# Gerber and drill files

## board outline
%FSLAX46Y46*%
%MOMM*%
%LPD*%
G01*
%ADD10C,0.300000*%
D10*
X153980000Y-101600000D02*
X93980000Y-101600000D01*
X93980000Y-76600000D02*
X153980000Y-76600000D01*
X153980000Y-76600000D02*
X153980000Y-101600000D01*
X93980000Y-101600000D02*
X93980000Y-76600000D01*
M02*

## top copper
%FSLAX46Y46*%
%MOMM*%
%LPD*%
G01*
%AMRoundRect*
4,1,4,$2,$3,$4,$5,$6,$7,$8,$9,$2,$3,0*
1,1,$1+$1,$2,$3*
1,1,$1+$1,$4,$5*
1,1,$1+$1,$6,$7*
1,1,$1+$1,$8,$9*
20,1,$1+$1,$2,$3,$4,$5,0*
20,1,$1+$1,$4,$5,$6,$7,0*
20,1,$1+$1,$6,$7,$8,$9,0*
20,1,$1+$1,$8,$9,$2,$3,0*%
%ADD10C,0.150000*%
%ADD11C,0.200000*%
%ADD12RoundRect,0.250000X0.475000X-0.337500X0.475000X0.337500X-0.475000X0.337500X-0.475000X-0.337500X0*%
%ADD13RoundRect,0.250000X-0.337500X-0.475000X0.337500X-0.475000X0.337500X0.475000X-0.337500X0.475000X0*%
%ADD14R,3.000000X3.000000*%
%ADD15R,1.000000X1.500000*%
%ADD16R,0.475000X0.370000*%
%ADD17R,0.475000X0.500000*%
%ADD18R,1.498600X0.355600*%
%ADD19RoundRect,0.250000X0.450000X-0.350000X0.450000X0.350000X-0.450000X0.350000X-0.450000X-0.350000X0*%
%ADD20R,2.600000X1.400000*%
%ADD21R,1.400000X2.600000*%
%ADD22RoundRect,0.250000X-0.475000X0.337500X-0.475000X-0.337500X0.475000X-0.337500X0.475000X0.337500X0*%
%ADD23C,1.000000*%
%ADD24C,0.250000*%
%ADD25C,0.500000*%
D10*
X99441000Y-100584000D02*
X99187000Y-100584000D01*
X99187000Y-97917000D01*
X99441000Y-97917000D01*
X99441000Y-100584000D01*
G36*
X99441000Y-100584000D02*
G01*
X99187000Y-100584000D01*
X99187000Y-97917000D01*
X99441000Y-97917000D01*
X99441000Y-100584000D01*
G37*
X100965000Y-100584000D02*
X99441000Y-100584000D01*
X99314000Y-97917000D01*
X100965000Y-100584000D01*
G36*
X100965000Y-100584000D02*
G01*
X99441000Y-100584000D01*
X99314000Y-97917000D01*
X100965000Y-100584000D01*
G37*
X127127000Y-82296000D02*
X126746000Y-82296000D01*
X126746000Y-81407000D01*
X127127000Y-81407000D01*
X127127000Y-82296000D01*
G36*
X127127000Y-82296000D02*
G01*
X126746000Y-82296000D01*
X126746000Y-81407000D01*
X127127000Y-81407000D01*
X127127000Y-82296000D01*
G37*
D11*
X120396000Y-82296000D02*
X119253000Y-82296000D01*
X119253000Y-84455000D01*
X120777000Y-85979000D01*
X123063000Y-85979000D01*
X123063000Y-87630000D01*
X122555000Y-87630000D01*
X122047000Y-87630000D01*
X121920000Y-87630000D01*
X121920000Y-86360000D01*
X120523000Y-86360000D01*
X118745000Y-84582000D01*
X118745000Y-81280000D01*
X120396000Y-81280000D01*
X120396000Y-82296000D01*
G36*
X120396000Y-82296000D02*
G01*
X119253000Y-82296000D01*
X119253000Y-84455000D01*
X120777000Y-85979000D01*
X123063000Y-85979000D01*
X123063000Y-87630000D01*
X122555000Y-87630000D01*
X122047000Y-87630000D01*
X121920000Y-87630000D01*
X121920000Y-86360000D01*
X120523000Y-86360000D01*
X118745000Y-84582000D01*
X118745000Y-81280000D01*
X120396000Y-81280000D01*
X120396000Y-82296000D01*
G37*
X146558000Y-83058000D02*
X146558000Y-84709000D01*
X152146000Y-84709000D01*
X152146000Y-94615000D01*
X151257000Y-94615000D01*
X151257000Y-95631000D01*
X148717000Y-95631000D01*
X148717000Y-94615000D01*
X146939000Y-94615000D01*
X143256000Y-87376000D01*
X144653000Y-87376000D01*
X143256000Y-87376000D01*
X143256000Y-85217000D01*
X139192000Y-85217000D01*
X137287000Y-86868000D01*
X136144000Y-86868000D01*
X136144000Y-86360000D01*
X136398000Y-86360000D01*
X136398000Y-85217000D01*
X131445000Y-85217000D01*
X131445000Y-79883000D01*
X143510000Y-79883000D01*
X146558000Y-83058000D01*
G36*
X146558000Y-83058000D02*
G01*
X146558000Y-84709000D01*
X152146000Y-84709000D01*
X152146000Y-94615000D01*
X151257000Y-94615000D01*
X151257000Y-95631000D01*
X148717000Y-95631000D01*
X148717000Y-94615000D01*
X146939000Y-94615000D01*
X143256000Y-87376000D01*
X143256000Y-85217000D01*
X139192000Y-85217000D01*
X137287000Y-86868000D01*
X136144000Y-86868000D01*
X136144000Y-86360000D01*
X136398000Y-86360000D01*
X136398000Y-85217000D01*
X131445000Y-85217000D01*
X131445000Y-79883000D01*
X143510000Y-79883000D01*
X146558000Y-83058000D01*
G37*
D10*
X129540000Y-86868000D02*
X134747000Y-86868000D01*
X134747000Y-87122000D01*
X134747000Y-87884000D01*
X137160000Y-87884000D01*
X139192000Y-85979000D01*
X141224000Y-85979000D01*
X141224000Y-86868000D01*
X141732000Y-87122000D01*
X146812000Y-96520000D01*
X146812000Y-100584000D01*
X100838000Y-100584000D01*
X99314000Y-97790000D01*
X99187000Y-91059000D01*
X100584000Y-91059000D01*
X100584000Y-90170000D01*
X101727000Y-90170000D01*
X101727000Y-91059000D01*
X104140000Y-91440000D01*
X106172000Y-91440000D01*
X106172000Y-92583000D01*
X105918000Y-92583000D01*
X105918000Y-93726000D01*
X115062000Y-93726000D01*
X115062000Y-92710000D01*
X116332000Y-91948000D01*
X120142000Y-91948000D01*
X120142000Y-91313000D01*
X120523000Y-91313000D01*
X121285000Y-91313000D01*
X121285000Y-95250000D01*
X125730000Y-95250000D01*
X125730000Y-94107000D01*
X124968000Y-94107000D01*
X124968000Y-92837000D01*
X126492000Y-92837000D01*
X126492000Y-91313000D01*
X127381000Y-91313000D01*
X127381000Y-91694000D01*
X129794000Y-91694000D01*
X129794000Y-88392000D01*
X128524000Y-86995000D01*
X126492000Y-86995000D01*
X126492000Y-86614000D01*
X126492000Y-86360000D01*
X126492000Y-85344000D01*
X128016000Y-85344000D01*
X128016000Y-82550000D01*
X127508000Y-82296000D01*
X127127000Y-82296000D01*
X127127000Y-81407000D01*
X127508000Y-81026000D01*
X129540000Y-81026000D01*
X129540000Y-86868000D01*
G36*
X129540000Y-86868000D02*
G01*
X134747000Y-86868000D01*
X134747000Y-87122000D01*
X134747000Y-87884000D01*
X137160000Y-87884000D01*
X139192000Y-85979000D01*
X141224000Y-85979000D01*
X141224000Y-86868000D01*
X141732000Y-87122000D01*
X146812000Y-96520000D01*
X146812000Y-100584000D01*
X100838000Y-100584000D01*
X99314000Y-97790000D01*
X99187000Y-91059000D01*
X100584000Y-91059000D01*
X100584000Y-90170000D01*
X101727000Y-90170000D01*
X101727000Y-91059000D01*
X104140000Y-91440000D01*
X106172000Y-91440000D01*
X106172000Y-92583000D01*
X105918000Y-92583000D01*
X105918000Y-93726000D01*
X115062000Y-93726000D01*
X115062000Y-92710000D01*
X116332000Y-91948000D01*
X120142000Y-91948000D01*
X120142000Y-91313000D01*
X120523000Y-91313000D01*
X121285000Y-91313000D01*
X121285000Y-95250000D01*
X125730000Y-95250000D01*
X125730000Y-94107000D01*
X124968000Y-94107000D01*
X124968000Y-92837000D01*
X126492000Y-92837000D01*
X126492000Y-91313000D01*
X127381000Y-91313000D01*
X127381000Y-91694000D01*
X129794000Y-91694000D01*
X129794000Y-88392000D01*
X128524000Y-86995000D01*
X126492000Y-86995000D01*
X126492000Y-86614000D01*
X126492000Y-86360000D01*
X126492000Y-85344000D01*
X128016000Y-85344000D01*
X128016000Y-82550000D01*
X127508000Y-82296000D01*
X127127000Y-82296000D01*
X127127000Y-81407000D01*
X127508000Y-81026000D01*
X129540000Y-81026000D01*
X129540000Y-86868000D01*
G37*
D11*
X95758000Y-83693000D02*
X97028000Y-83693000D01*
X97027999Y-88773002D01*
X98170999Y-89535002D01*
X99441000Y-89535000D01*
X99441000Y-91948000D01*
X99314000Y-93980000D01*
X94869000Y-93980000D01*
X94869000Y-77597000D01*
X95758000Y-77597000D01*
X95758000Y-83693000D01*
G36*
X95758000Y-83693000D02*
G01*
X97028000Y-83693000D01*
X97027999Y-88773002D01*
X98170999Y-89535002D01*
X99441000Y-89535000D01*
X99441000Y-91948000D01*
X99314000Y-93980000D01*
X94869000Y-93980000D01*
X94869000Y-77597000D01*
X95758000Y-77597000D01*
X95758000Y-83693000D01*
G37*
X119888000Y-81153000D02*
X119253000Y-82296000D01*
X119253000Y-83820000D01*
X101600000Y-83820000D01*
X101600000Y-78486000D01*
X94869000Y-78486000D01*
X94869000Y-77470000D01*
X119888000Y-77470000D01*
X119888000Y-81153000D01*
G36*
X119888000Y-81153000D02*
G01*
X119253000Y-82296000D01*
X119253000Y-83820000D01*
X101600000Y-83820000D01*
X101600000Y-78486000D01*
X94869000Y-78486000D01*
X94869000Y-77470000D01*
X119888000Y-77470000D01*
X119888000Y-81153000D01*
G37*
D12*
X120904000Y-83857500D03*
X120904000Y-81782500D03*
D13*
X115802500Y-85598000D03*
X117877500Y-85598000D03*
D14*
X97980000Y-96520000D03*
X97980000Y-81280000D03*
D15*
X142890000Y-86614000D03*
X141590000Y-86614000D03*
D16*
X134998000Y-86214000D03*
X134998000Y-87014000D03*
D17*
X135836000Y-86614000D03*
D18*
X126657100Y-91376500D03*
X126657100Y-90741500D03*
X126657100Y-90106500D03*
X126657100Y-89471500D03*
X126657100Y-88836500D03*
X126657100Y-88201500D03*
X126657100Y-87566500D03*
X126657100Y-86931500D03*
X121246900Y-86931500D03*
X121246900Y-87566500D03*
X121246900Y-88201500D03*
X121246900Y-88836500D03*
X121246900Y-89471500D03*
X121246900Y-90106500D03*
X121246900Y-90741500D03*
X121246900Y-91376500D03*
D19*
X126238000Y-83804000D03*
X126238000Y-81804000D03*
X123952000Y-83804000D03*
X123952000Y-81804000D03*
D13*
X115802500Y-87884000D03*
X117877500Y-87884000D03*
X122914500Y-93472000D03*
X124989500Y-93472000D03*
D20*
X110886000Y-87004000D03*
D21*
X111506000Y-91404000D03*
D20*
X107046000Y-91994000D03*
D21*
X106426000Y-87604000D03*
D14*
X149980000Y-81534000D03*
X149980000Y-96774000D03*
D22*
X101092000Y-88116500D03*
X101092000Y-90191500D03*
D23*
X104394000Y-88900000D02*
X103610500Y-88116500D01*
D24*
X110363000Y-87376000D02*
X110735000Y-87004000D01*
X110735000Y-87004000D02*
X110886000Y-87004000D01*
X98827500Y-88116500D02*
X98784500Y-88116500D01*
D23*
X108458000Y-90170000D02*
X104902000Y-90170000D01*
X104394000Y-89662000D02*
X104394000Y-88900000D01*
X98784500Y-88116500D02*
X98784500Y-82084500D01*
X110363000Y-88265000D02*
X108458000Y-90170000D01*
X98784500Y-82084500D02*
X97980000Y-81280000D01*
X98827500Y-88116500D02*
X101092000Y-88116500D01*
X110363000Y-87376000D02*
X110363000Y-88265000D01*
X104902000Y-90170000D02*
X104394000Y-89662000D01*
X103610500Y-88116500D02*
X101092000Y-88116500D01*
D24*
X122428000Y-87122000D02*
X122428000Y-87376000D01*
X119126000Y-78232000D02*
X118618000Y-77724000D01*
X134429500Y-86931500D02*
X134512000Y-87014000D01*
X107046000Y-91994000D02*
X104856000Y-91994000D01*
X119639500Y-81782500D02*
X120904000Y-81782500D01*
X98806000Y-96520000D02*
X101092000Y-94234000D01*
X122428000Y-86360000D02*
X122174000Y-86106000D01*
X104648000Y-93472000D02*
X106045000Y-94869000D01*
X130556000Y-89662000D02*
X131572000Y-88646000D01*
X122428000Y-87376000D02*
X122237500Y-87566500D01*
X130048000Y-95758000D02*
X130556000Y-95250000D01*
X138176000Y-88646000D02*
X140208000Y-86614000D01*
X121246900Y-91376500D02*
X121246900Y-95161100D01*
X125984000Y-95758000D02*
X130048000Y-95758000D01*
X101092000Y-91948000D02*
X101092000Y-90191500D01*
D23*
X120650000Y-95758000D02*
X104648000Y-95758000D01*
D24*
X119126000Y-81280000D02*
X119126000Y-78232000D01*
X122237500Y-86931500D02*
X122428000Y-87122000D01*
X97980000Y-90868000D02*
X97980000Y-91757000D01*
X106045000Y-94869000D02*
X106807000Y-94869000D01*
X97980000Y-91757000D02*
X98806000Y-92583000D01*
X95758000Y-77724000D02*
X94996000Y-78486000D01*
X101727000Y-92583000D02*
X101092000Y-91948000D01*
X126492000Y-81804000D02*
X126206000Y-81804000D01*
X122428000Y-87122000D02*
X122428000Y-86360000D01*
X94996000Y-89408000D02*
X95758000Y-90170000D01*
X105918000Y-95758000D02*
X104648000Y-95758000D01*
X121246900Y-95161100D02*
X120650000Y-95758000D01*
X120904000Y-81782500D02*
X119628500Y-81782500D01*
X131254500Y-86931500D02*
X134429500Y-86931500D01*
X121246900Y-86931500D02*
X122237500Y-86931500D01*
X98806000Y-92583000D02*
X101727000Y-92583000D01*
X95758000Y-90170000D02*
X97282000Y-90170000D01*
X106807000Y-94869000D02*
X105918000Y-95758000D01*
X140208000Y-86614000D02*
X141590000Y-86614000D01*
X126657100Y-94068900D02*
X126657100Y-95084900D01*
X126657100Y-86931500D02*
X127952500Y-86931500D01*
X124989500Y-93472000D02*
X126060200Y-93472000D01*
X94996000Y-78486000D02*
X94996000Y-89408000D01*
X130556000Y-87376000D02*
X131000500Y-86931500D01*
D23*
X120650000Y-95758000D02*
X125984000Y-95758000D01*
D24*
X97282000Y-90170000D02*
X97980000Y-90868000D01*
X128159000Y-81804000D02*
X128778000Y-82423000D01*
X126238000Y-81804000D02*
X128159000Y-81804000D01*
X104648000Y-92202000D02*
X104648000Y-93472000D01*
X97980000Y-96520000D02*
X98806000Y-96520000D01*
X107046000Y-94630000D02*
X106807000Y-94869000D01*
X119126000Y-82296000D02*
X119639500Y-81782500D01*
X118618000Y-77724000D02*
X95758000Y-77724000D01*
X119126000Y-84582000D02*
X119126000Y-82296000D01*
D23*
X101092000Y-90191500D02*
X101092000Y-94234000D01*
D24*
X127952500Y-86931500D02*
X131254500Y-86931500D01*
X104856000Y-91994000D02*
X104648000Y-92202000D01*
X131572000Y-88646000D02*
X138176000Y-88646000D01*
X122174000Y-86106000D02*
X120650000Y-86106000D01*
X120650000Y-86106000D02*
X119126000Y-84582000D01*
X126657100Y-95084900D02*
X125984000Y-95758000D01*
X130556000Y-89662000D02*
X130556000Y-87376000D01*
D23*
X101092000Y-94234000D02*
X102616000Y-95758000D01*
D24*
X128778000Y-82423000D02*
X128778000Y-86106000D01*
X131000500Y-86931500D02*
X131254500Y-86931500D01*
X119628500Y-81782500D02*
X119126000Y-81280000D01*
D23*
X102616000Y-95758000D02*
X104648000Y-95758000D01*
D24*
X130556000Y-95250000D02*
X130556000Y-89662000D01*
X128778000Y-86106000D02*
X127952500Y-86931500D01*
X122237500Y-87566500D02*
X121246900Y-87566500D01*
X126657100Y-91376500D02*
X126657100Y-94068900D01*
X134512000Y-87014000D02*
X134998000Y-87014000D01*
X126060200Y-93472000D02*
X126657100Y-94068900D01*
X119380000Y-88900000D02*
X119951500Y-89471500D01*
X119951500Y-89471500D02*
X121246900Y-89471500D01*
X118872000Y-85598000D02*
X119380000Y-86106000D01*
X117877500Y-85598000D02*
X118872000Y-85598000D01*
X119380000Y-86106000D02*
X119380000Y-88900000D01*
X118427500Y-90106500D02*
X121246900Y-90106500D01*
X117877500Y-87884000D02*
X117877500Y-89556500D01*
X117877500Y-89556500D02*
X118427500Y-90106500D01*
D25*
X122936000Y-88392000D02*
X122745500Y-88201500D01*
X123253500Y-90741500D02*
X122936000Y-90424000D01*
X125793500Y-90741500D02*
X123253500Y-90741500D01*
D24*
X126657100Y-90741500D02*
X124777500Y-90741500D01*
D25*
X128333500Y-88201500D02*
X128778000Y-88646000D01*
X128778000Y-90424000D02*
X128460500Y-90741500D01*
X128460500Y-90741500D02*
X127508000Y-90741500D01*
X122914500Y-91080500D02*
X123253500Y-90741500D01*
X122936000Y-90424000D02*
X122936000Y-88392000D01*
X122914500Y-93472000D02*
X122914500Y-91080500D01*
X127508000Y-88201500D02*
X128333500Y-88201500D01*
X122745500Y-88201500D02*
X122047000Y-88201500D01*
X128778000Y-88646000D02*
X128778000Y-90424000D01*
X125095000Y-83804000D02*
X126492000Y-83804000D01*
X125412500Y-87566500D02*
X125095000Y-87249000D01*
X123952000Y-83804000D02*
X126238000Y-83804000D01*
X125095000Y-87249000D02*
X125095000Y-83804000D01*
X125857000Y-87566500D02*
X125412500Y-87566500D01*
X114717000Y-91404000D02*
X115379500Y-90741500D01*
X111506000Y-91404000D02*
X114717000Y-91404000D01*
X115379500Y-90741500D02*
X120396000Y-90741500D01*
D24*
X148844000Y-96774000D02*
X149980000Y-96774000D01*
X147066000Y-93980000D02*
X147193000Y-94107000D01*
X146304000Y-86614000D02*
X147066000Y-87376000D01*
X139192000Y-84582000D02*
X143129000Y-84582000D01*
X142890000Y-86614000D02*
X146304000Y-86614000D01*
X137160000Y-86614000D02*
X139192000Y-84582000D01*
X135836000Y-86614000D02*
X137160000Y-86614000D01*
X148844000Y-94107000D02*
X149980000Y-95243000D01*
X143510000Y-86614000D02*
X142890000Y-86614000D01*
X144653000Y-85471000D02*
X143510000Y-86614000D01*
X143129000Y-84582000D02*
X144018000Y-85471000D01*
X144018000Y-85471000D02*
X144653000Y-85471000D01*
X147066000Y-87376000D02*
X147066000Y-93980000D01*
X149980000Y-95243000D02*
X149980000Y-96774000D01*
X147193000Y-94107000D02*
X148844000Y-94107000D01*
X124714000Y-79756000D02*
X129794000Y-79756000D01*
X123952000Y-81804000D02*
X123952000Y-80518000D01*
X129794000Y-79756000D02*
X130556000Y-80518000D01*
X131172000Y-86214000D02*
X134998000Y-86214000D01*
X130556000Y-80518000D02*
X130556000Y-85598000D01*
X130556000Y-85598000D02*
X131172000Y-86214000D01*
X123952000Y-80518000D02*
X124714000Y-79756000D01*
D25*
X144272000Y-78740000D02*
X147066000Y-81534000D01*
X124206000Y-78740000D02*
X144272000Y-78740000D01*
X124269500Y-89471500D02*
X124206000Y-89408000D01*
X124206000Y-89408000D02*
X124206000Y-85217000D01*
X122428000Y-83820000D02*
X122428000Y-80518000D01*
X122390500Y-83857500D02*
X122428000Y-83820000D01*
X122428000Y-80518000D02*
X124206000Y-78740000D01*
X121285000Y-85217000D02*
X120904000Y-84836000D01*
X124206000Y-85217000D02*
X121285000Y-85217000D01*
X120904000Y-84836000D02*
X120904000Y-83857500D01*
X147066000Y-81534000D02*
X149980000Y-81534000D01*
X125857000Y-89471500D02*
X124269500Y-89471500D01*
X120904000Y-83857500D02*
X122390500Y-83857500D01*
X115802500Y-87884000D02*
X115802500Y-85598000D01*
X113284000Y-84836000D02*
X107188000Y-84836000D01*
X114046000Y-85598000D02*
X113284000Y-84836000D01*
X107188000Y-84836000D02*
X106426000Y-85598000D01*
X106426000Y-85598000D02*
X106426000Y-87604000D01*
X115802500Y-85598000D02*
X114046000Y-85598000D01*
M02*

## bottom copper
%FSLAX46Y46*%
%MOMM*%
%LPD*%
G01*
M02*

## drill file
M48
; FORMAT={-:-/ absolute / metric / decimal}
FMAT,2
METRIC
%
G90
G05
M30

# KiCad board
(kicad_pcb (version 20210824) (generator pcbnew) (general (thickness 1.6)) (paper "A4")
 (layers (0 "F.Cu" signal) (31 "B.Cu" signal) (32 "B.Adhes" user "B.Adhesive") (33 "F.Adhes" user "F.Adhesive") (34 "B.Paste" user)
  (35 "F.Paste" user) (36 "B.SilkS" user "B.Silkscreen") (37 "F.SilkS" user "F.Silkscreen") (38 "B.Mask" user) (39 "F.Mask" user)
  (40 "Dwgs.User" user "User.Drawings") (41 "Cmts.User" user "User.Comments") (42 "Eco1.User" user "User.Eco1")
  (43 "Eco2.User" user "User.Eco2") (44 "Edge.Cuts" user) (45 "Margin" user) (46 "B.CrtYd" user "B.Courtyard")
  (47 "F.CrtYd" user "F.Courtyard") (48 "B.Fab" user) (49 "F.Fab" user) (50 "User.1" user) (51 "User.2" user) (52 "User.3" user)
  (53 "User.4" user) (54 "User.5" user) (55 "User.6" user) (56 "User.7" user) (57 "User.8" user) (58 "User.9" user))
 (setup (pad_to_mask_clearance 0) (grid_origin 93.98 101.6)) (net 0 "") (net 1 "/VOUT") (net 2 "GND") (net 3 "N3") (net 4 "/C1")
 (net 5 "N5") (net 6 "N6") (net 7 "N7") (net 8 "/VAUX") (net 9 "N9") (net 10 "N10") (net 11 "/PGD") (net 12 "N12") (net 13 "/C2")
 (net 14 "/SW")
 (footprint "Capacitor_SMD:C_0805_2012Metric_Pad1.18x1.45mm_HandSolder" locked (layer "F.Cu") (at 120.904 82.82 90)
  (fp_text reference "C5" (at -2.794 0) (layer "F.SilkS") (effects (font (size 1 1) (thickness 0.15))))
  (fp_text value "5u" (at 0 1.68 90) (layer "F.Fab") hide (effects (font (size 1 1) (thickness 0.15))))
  (pad "1" smd roundrect locked (at -1.0375 0 90) (size 1.175 1.45) (layers "F.Cu" "F.Paste" "F.Mask") (roundrect_rratio 0.2127659574)
   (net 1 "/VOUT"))
  (pad "2" smd roundrect locked (at 1.0375 0 90) (size 1.175 1.45) (layers "F.Cu" "F.Paste" "F.Mask") (roundrect_rratio 0.2127659574)
   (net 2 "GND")))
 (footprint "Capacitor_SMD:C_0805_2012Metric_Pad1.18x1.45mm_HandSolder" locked (layer "F.Cu") (at 116.84 85.598)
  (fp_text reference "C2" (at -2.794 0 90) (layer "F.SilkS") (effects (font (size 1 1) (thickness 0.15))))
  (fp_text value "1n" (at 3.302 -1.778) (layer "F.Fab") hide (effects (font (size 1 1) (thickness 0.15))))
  (pad "1" smd roundrect locked (at -1.0375 0) (size 1.175 1.45) (layers "F.Cu" "F.Paste" "F.Mask") (roundrect_rratio 0.2127659574)
   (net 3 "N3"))
  (pad "2" smd roundrect locked (at 1.0375 0) (size 1.175 1.45) (layers "F.Cu" "F.Paste" "F.Mask") (roundrect_rratio 0.2127659574)
   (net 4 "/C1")))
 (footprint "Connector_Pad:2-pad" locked (layer "F.Cu") (at 97.98 88.9 90)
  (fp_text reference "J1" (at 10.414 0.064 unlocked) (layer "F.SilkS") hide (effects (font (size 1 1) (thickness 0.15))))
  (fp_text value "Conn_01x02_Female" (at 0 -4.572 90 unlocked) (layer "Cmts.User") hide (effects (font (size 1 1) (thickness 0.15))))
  (pad "1" smd rect locked (at -7.62 0) (size 3 3) (layers "F.Cu" "F.Paste" "F.Mask") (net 2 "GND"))
  (pad "2" smd rect locked (at 7.62 0 180) (size 3 3) (layers "F.Cu" "F.Paste" "F.Mask") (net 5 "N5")))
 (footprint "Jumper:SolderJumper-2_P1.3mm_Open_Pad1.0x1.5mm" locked (layer "F.Cu") (at 142.24 86.614 180)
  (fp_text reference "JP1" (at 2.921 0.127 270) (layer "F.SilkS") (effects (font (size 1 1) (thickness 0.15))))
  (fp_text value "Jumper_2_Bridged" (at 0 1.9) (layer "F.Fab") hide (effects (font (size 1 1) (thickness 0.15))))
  (pad "1" smd rect locked (at -0.65 0 180) (size 1 1.5) (layers "F.Cu" "F.Mask") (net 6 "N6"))
  (pad "2" smd rect locked (at 0.65 0 180) (size 1 1.5) (layers "F.Cu" "F.Mask") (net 2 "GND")))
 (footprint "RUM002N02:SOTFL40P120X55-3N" (layer "F.Cu") (at 135.636 86.614)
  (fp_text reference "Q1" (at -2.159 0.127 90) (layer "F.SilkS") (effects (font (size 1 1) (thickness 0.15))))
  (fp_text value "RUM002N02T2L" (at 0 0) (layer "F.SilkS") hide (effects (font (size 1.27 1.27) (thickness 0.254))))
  (pad "1" smd rect (at -0.638 -0.4) (size 0.475 0.37) (layers "F.Cu" "F.Paste" "F.Mask") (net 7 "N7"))
  (pad "2" smd rect (at -0.638 0.4) (size 0.475 0.37) (layers "F.Cu" "F.Paste" "F.Mask") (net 2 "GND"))
  (pad "3" smd rect (at 0.2 0) (size 0.475 0.5) (layers "F.Cu" "F.Paste" "F.Mask") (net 6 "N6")))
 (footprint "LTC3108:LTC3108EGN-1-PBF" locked (layer "F.Cu") (at 123.952 89.154 180)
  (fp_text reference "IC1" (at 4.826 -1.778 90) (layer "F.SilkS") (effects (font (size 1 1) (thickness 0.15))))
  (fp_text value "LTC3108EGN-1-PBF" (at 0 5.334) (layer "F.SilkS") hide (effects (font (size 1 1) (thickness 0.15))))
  (pad "1" smd rect locked (at -2.7051 -2.2225 180) (size 1.4986 0.3556) (layers "F.Cu" "F.Paste" "F.Mask") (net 2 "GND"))
  (pad "2" smd rect locked (at -2.7051 -1.5875 180) (size 1.4986 0.3556) (layers "F.Cu" "F.Paste" "F.Mask") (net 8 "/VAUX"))
  (pad "3" smd rect locked (at -2.7051 -0.9525 180) (size 1.4986 0.3556) (layers "F.Cu" "F.Paste" "F.Mask") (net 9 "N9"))
  (pad "4" smd rect locked (at -2.7051 -0.3175 180) (size 1.4986 0.3556) (layers "F.Cu" "F.Paste" "F.Mask") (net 1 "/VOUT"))
  (pad "5" smd rect locked (at -2.7051 0.3175 180) (size 1.4986 0.3556) (layers "F.Cu" "F.Paste" "F.Mask") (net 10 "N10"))
  (pad "6" smd rect locked (at -2.7051 0.9525 180) (size 1.4986 0.3556) (layers "F.Cu" "F.Paste" "F.Mask") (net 8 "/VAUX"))
  (pad "7" smd rect locked (at -2.7051 1.5875 180) (size 1.4986 0.3556) (layers "F.Cu" "F.Paste" "F.Mask") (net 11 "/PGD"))
  (pad "8" smd rect locked (at -2.7051 2.2225 180) (size 1.4986 0.3556) (layers "F.Cu" "F.Paste" "F.Mask") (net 2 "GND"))
  (pad "9" smd rect locked (at 2.7051 2.2225 180) (size 1.4986 0.3556) (layers "F.Cu" "F.Paste" "F.Mask") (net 2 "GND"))
  (pad "10" smd rect locked (at 2.7051 1.5875 180) (size 1.4986 0.3556) (layers "F.Cu" "F.Paste" "F.Mask") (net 2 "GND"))
  (pad "11" smd rect locked (at 2.7051 0.9525 180) (size 1.4986 0.3556) (layers "F.Cu" "F.Paste" "F.Mask") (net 8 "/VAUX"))
  (pad "12" smd rect locked (at 2.7051 0.3175 180) (size 1.4986 0.3556) (layers "F.Cu" "F.Paste" "F.Mask") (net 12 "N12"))
  (pad "13" smd rect locked (at 2.7051 -0.3175 180) (size 1.4986 0.3556) (layers "F.Cu" "F.Paste" "F.Mask") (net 4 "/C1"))
  (pad "14" smd rect locked (at 2.7051 -0.9525 180) (size 1.4986 0.3556) (layers "F.Cu" "F.Paste" "F.Mask") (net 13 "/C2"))
  (pad "15" smd rect locked (at 2.7051 -1.5875 180) (size 1.4986 0.3556) (layers "F.Cu" "F.Paste" "F.Mask") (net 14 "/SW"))
  (pad "16" smd rect locked (at 2.7051 -2.2225 180) (size 1.4986 0.3556) (layers "F.Cu" "F.Paste" "F.Mask") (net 2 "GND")))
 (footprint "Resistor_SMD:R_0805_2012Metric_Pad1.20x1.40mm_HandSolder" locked (layer "F.Cu") (at 126.238 82.804 90)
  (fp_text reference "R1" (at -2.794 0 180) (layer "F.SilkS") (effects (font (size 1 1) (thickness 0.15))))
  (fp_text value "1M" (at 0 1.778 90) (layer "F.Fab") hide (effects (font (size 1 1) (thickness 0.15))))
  (pad "1" smd roundrect locked (at -1 0 90) (size 1.2 1.4) (layers "F.Cu" "F.Paste" "F.Mask") (roundrect_rratio 0.2083333333)
   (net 11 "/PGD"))
  (pad "2" smd roundrect locked (at 1 0 90) (size 1.2 1.4) (layers "F.Cu" "F.Paste" "F.Mask") (roundrect_rratio 0.2083333333) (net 2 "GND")))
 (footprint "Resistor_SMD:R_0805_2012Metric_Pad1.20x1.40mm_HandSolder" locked (layer "F.Cu") (at 123.952 82.804 90)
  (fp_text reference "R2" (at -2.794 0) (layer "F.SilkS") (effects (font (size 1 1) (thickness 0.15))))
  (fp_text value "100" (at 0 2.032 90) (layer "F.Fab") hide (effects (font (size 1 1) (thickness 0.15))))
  (pad "1" smd roundrect locked (at -1 0 90) (size 1.2 1.4) (layers "F.Cu" "F.Paste" "F.Mask") (roundrect_rratio 0.2083333333)
   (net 11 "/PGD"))
  (pad "2" smd roundrect locked (at 1 0 90) (size 1.2 1.4) (layers "F.Cu" "F.Paste" "F.Mask") (roundrect_rratio 0.2083333333) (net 7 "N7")))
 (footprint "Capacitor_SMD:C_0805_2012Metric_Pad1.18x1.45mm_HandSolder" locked (layer "F.Cu") (at 116.84 87.884)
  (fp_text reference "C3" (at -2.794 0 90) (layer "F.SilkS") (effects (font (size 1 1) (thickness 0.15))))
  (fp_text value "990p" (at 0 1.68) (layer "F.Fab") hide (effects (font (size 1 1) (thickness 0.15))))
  (pad "1" smd roundrect locked (at -1.0375 0) (size 1.175 1.45) (layers "F.Cu" "F.Paste" "F.Mask") (roundrect_rratio 0.2127659574)
   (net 3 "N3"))
  (pad "2" smd roundrect locked (at 1.0375 0) (size 1.175 1.45) (layers "F.Cu" "F.Paste" "F.Mask") (roundrect_rratio 0.2127659574)
   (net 13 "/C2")))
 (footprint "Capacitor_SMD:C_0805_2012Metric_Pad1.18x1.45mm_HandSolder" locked (layer "F.Cu") (at 123.952 93.472)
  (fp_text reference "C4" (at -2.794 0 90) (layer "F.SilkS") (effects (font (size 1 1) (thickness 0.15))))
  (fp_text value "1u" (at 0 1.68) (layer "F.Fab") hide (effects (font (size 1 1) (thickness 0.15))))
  (pad "1" smd roundrect locked (at -1.0375 0) (size 1.175 1.45) (layers "F.Cu" "F.Paste" "F.Mask") (roundrect_rratio 0.2127659574)
   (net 8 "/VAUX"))
  (pad "2" smd roundrect locked (at 1.0375 0) (size 1.175 1.45) (layers "F.Cu" "F.Paste" "F.Mask") (roundrect_rratio 0.2127659574)
   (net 2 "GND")))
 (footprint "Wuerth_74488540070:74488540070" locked (layer "F.Cu") (at 108.966 89.154 180)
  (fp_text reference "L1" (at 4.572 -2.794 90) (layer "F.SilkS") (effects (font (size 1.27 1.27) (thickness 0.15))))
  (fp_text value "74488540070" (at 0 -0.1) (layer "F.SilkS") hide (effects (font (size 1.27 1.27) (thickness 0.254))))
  (pad "1" smd rect locked (at -1.92 2.15 270) (size 1.4 2.6) (layers "F.Cu" "F.Paste" "F.Mask") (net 5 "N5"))
  (pad "2" smd rect locked (at -2.54 -2.25 180) (size 1.4 2.6) (layers "F.Cu" "F.Paste" "F.Mask") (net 14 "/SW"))
  (pad "3" smd rect locked (at 1.92 -2.84 270) (size 1.4 2.6) (layers "F.Cu" "F.Paste" "F.Mask") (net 2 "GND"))
  (pad "4" smd rect locked (at 2.54 1.55 180) (size 1.4 2.6) (layers "F.Cu" "F.Paste" "F.Mask") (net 3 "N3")))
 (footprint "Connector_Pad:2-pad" (layer "F.Cu") (at 149.98 89.154 -90)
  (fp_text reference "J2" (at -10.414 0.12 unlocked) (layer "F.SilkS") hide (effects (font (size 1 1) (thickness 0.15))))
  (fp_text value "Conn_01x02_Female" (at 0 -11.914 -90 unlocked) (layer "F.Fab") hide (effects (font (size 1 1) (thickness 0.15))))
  (pad "1" smd rect (at -7.62 0 270) (size 3 3) (layers "F.Cu" "F.Paste" "F.Mask") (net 1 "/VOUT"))
  (pad "2" smd rect (at 7.62 0 270) (size 3 3) (layers "F.Cu" "F.Paste" "F.Mask") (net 6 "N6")))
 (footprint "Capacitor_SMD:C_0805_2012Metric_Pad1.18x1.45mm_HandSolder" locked (layer "F.Cu") (at 101.092 89.154 -90)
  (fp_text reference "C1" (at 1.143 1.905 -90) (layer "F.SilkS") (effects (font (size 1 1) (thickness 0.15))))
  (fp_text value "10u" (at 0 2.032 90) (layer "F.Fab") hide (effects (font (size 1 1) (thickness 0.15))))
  (pad "1" smd roundrect locked (at -1.0375 0 270) (size 1.175 1.45) (layers "F.Cu" "F.Paste" "F.Mask") (roundrect_rratio 0.2127659574)
   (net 5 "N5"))
  (pad "2" smd roundrect locked (at 1.0375 0 270) (size 1.175 1.45) (layers "F.Cu" "F.Paste" "F.Mask") (roundrect_rratio 0.2127659574)
   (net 2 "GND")))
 (gr_poly (pts (xy 99.441 100.584) (xy 99.187 100.584) (xy 99.187 97.917) (xy 99.441 97.917)) (layer "F.Cu") (width 0.15) (fill solid))
 (gr_poly (pts (xy 100.965 100.584) (xy 99.441 100.584) (xy 99.314 97.917)) (layer "F.Cu") (width 0.15) (fill solid))
 (gr_poly (pts (xy 127.127 82.296) (xy 126.746 82.296) (xy 126.746 81.407) (xy 127.127 81.407)) (layer "F.Cu") (width 0.15) (fill solid))
 (gr_poly
  (pts (xy 120.396 82.296) (xy 119.253 82.296) (xy 119.253 84.455) (xy 120.777 85.979) (xy 123.063 85.979) (xy 123.063 87.63)
   (xy 122.555 87.63) (xy 122.047 87.63) (xy 121.92 87.63) (xy 121.92 86.36) (xy 120.523 86.36) (xy 118.745 84.582) (xy 118.745 81.28)
   (xy 120.396 81.28))
  (layer "F.Cu") (width 0.2) (fill solid))
 (gr_poly
  (pts (xy 146.558 83.058) (xy 146.558 84.709) (xy 152.146 84.709) (xy 152.146 94.615) (xy 151.257 94.615) (xy 151.257 95.631)
   (xy 148.717 95.631) (xy 148.717 94.615) (xy 146.939 94.615) (xy 143.256 87.376) (xy 144.653 87.376) (xy 143.256 87.376)
   (xy 143.256 85.217) (xy 139.192 85.217) (xy 137.287 86.868) (xy 136.144 86.868) (xy 136.144 86.36) (xy 136.398 86.36) (xy 136.398 85.217)
   (xy 131.445 85.217) (xy 131.445 79.883) (xy 143.51 79.883))
  (layer "F.Cu") (width 0.2) (fill solid))
 (gr_poly
  (pts (xy 129.54 86.868) (xy 134.747 86.868) (xy 134.747 87.122) (xy 134.747 87.884) (xy 137.16 87.884) (xy 139.192 85.979)
   (xy 141.224 85.979) (xy 141.224 86.868) (xy 141.732 87.122) (xy 146.812 96.52) (xy 146.812 100.584) (xy 100.838 100.584)
   (xy 99.314 97.79) (xy 99.187 91.059) (xy 100.584 91.059) (xy 100.584 90.17) (xy 101.727 90.17) (xy 101.727 91.059) (xy 104.14 91.44)
   (xy 106.172 91.44) (xy 106.172 92.583) (xy 105.918 92.583) (xy 105.918 93.726) (xy 115.062 93.726) (xy 115.062 92.71) (xy 116.332 91.948)
   (xy 120.142 91.948) (xy 120.142 91.313) (xy 120.523 91.313) (xy 121.285 91.313) (xy 121.285 95.25) (xy 125.73 95.25) (xy 125.73 94.107)
   (xy 124.968 94.107) (xy 124.968 92.837) (xy 126.492 92.837) (xy 126.492 91.313) (xy 127.381 91.313) (xy 127.381 91.694)
   (xy 129.794 91.694) (xy 129.794 88.392) (xy 128.524 86.995) (xy 126.492 86.995) (xy 126.492 86.614) (xy 126.492 86.36)
   (xy 126.492 85.344) (xy 128.016 85.344) (xy 128.016 82.55) (xy 127.508 82.296) (xy 127.127 82.296) (xy 127.127 81.407)
   (xy 127.508 81.026) (xy 129.54 81.026))
  (layer "F.Cu") (width 0.15) (fill solid))
 (gr_poly
  (pts (xy 95.758 83.693) (xy 97.028 83.693) (xy 97.027999 88.773002) (xy 98.170999 89.535002) (xy 99.441 89.535) (xy 99.441 91.948)
   (xy 99.314 93.98) (xy 94.869 93.98) (xy 94.869 77.597) (xy 95.758 77.597))
  (layer "F.Cu") (width 0.2) (fill solid))
 (gr_poly
  (pts (xy 119.888 81.153) (xy 119.253 82.296) (xy 119.253 83.82) (xy 101.6 83.82) (xy 101.6 78.486) (xy 94.869 78.486) (xy 94.869 77.47)
   (xy 119.888 77.47))
  (layer "F.Cu") (width 0.2) (fill solid))
 (gr_line locked (start 153.98 101.6) (end 93.98 101.6) (layer "Edge.Cuts") (width 0.3))
 (gr_line locked (start 93.98 76.6) (end 153.98 76.6) (layer "Edge.Cuts") (width 0.3))
 (gr_line locked (start 153.98 76.6) (end 153.98 101.6) (layer "Edge.Cuts") (width 0.3))
 (gr_line locked (start 93.98 101.6) (end 93.98 76.6) (layer "Edge.Cuts") (width 0.3))
 (segment (start 104.394 88.9) (end 103.6105 88.1165) (width 1) (layer "F.Cu") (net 5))
 (segment (start 110.363 87.376) (end 110.735 87.004) (width 0.25) (layer "F.Cu") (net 5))
 (segment (start 110.735 87.004) (end 110.886 87.004) (width 0.25) (layer "F.Cu") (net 5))
 (segment (start 98.8275 88.1165) (end 98.7845 88.1165) (width 0.25) (layer "F.Cu") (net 5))
 (segment (start 108.458 90.17) (end 104.902 90.17) (width 1) (layer "F.Cu") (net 5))
 (segment (start 104.394 89.662) (end 104.394 88.9) (width 1) (layer "F.Cu") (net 5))
 (segment (start 98.7845 88.1165) (end 98.7845 82.0845) (width 1) (layer "F.Cu") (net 5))
 (segment (start 110.363 88.265) (end 108.458 90.17) (width 1) (layer "F.Cu") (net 5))
 (segment (start 98.7845 82.0845) (end 97.98 81.28) (width 1) (layer "F.Cu") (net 5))
 (segment (start 98.8275 88.1165) (end 101.092 88.1165) (width 1) (layer "F.Cu") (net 5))
 (segment (start 110.363 87.376) (end 110.363 88.265) (width 1) (layer "F.Cu") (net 5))
 (segment (start 104.902 90.17) (end 104.394 89.662) (width 1) (layer "F.Cu") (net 5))
 (segment (start 103.6105 88.1165) (end 101.092 88.1165) (width 1) (layer "F.Cu") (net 5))
 (segment (start 122.428 87.122) (end 122.428 87.376) (width 0.25) (layer "F.Cu") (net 2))
 (segment (start 119.126 78.232) (end 118.618 77.724) (width 0.25) (layer "F.Cu") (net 2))
 (segment (start 134.4295 86.9315) (end 134.512 87.014) (width 0.25) (layer "F.Cu") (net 2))
 (segment (start 107.046 91.994) (end 104.856 91.994) (width 0.25) (layer "F.Cu") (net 2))
 (segment (start 119.6395 81.7825) (end 120.904 81.7825) (width 0.25) (layer "F.Cu") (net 2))
 (segment (start 98.806 96.52) (end 101.092 94.234) (width 0.25) (layer "F.Cu") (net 2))
 (segment (start 122.428 86.36) (end 122.174 86.106) (width 0.25) (layer "F.Cu") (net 2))
 (segment (start 104.648 93.472) (end 106.045 94.869) (width 0.25) (layer "F.Cu") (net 2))
 (segment (start 130.556 89.662) (end 131.572 88.646) (width 0.25) (layer "F.Cu") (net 2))
 (segment (start 122.428 87.376) (end 122.2375 87.5665) (width 0.25) (layer "F.Cu") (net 2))
 (segment (start 130.048 95.758) (end 130.556 95.25) (width 0.25) (layer "F.Cu") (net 2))
 (segment (start 138.176 88.646) (end 140.208 86.614) (width 0.25) (layer "F.Cu") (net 2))
 (segment (start 121.2469 91.3765) (end 121.2469 95.1611) (width 0.25) (layer "F.Cu") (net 2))
 (segment (start 125.984 95.758) (end 130.048 95.758) (width 0.25) (layer "F.Cu") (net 2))
 (segment (start 101.092 91.948) (end 101.092 90.1915) (width 0.25) (layer "F.Cu") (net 2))
 (segment (start 120.65 95.758) (end 104.648 95.758) (width 1) (layer "F.Cu") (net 2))
 (segment (start 119.126 81.28) (end 119.126 78.232) (width 0.25) (layer "F.Cu") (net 2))
 (segment (start 122.2375 86.9315) (end 122.428 87.122) (width 0.25) (layer "F.Cu") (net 2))
 (segment (start 97.98 90.868) (end 97.98 91.757) (width 0.25) (layer "F.Cu") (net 2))
 (segment (start 106.045 94.869) (end 106.807 94.869) (width 0.25) (layer "F.Cu") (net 2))
 (segment (start 97.98 91.757) (end 98.806 92.583) (width 0.25) (layer "F.Cu") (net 2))
 (segment (start 95.758 77.724) (end 94.996 78.486) (width 0.25) (layer "F.Cu") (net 2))
 (segment (start 101.727 92.583) (end 101.092 91.948) (width 0.25) (layer "F.Cu") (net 2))
 (segment (start 126.492 81.804) (end 126.206 81.804) (width 0.25) (layer "F.Cu") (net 2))
 (segment (start 122.428 87.122) (end 122.428 86.36) (width 0.25) (layer "F.Cu") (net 2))
 (segment (start 94.996 89.408) (end 95.758 90.17) (width 0.25) (layer "F.Cu") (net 2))
 (segment (start 105.918 95.758) (end 104.648 95.758) (width 0.25) (layer "F.Cu") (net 2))
 (segment (start 121.2469 95.1611) (end 120.65 95.758) (width 0.25) (layer "F.Cu") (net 2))
 (segment (start 120.904 81.7825) (end 119.6285 81.7825) (width 0.25) (layer "F.Cu") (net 2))
 (segment (start 131.2545 86.9315) (end 134.4295 86.9315) (width 0.25) (layer "F.Cu") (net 2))
 (segment (start 121.2469 86.9315) (end 122.2375 86.9315) (width 0.25) (layer "F.Cu") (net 2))
 (segment (start 98.806 92.583) (end 101.727 92.583) (width 0.25) (layer "F.Cu") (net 2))
 (segment (start 95.758 90.17) (end 97.282 90.17) (width 0.25) (layer "F.Cu") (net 2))
 (segment (start 106.807 94.869) (end 105.918 95.758) (width 0.25) (layer "F.Cu") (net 2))
 (segment (start 140.208 86.614) (end 141.59 86.614) (width 0.25) (layer "F.Cu") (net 2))
 (segment (start 126.6571 94.0689) (end 126.6571 95.0849) (width 0.25) (layer "F.Cu") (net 2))
 (segment (start 126.6571 86.9315) (end 127.9525 86.9315) (width 0.25) (layer "F.Cu") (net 2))
 (segment (start 124.9895 93.472) (end 126.0602 93.472) (width 0.25) (layer "F.Cu") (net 2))
 (segment (start 94.996 78.486) (end 94.996 89.408) (width 0.25) (layer "F.Cu") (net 2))
 (segment (start 130.556 87.376) (end 131.0005 86.9315) (width 0.25) (layer "F.Cu") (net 2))
 (segment (start 120.65 95.758) (end 125.984 95.758) (width 1) (layer "F.Cu") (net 2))
 (segment (start 97.282 90.17) (end 97.98 90.868) (width 0.25) (layer "F.Cu") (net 2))
 (segment (start 128.159 81.804) (end 128.778 82.423) (width 0.25) (layer "F.Cu") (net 2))
 (segment (start 126.238 81.804) (end 128.159 81.804) (width 0.25) (layer "F.Cu") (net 2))
 (segment (start 104.648 92.202) (end 104.648 93.472) (width 0.25) (layer "F.Cu") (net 2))
 (segment (start 97.98 96.52) (end 98.806 96.52) (width 0.25) (layer "F.Cu") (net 2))
 (segment (start 107.046 94.63) (end 106.807 94.869) (width 0.25) (layer "F.Cu") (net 2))
 (segment (start 119.126 82.296) (end 119.6395 81.7825) (width 0.25) (layer "F.Cu") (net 2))
 (segment (start 118.618 77.724) (end 95.758 77.724) (width 0.25) (layer "F.Cu") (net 2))
 (segment (start 119.126 84.582) (end 119.126 82.296) (width 0.25) (layer "F.Cu") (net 2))
 (segment (start 101.092 90.1915) (end 101.092 94.234) (width 1) (layer "F.Cu") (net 2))
 (segment (start 127.9525 86.9315) (end 131.2545 86.9315) (width 0.25) (layer "F.Cu") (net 2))
 (segment (start 104.856 91.994) (end 104.648 92.202) (width 0.25) (layer "F.Cu") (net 2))
 (segment (start 131.572 88.646) (end 138.176 88.646) (width 0.25) (layer "F.Cu") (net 2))
 (segment (start 122.174 86.106) (end 120.65 86.106) (width 0.25) (layer "F.Cu") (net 2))
 (segment (start 120.65 86.106) (end 119.126 84.582) (width 0.25) (layer "F.Cu") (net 2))
 (segment (start 126.6571 95.0849) (end 125.984 95.758) (width 0.25) (layer "F.Cu") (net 2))
 (segment (start 130.556 89.662) (end 130.556 87.376) (width 0.25) (layer "F.Cu") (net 2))
 (segment (start 101.092 94.234) (end 102.616 95.758) (width 1) (layer "F.Cu") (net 2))
 (segment (start 128.778 82.423) (end 128.778 86.106) (width 0.25) (layer "F.Cu") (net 2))
 (segment (start 131.0005 86.9315) (end 131.2545 86.9315) (width 0.25) (layer "F.Cu") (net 2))
 (segment (start 119.6285 81.7825) (end 119.126 81.28) (width 0.25) (layer "F.Cu") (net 2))
 (segment (start 102.616 95.758) (end 104.648 95.758) (width 1) (layer "F.Cu") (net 2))
 (segment (start 130.556 95.25) (end 130.556 89.662) (width 0.25) (layer "F.Cu") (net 2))
 (segment (start 128.778 86.106) (end 127.9525 86.9315) (width 0.25) (layer "F.Cu") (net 2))
 (segment (start 122.2375 87.5665) (end 121.2469 87.5665) (width 0.25) (layer "F.Cu") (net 2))
 (segment (start 126.6571 91.3765) (end 126.6571 94.0689) (width 0.25) (layer "F.Cu") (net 2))
 (segment (start 134.512 87.014) (end 134.998 87.014) (width 0.25) (layer "F.Cu") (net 2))
 (segment (start 126.0602 93.472) (end 126.6571 94.0689) (width 0.25) (layer "F.Cu") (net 2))
 (segment (start 119.38 88.9) (end 119.9515 89.4715) (width 0.25) (layer "F.Cu") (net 4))
 (segment (start 119.9515 89.4715) (end 121.2469 89.4715) (width 0.25) (layer "F.Cu") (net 4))
 (segment (start 118.872 85.598) (end 119.38 86.106) (width 0.25) (layer "F.Cu") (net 4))
 (segment (start 117.8775 85.598) (end 118.872 85.598) (width 0.25) (layer "F.Cu") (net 4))
 (segment (start 119.38 86.106) (end 119.38 88.9) (width 0.25) (layer "F.Cu") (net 4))
 (segment (start 118.4275 90.1065) (end 121.2469 90.1065) (width 0.25) (layer "F.Cu") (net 13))
 (segment (start 117.8775 87.884) (end 117.8775 89.5565) (width 0.25) (layer "F.Cu") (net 13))
 (segment (start 117.8775 89.5565) (end 118.4275 90.1065) (width 0.25) (layer "F.Cu") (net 13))
 (segment (start 122.936 88.392) (end 122.7455 88.2015) (width 0.5) (layer "F.Cu") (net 8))
 (segment (start 123.2535 90.7415) (end 122.936 90.424) (width 0.5) (layer "F.Cu") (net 8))
 (segment (start 125.7935 90.7415) (end 123.2535 90.7415) (width 0.5) (layer "F.Cu") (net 8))
 (segment (start 126.6571 90.7415) (end 124.7775 90.7415) (width 0.25) (layer "F.Cu") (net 8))
 (segment (start 128.3335 88.2015) (end 128.778 88.646) (width 0.5) (layer "F.Cu") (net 8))
 (segment (start 128.778 90.424) (end 128.4605 90.7415) (width 0.5) (layer "F.Cu") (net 8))
 (segment (start 128.4605 90.7415) (end 127.508 90.7415) (width 0.5) (layer "F.Cu") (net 8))
 (segment (start 122.9145 91.0805) (end 123.2535 90.7415) (width 0.5) (layer "F.Cu") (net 8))
 (segment (start 122.936 90.424) (end 122.936 88.392) (width 0.5) (layer "F.Cu") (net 8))
 (segment (start 122.9145 93.472) (end 122.9145 91.0805) (width 0.5) (layer "F.Cu") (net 8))
 (segment (start 127.508 88.2015) (end 128.3335 88.2015) (width 0.5) (layer "F.Cu") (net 8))
 (segment (start 122.7455 88.2015) (end 122.047 88.2015) (width 0.5) (layer "F.Cu") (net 8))
 (segment (start 128.778 88.646) (end 128.778 90.424) (width 0.5) (layer "F.Cu") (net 8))
 (segment (start 125.095 83.804) (end 126.492 83.804) (width 0.5) (layer "F.Cu") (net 11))
 (segment (start 125.4125 87.5665) (end 125.095 87.249) (width 0.5) (layer "F.Cu") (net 11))
 (segment (start 123.952 83.804) (end 126.238 83.804) (width 0.5) (layer "F.Cu") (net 11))
 (segment (start 125.095 87.249) (end 125.095 83.804) (width 0.5) (layer "F.Cu") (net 11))
 (segment (start 125.857 87.5665) (end 125.4125 87.5665) (width 0.5) (layer "F.Cu") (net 11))
 (segment (start 114.717 91.404) (end 115.3795 90.7415) (width 0.5) (layer "F.Cu") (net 14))
 (segment (start 111.506 91.404) (end 114.717 91.404) (width 0.5) (layer "F.Cu") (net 14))
 (segment (start 115.3795 90.7415) (end 120.396 90.7415) (width 0.5) (layer "F.Cu") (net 14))
 (segment (start 148.844 96.774) (end 149.98 96.774) (width 0.25) (layer "F.Cu") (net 6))
 (segment (start 147.066 93.98) (end 147.193 94.107) (width 0.25) (layer "F.Cu") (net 6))
 (segment (start 146.304 86.614) (end 147.066 87.376) (width 0.25) (layer "F.Cu") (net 6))
 (segment (start 139.192 84.582) (end 143.129 84.582) (width 0.25) (layer "F.Cu") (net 6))
 (segment (start 142.89 86.614) (end 146.304 86.614) (width 0.25) (layer "F.Cu") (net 6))
 (segment (start 137.16 86.614) (end 139.192 84.582) (width 0.25) (layer "F.Cu") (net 6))
 (segment (start 135.836 86.614) (end 137.16 86.614) (width 0.25) (layer "F.Cu") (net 6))
 (segment (start 148.844 94.107) (end 149.98 95.243) (width 0.25) (layer "F.Cu") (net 6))
 (segment (start 143.51 86.614) (end 142.89 86.614) (width 0.25) (layer "F.Cu") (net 6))
 (segment (start 144.653 85.471) (end 143.51 86.614) (width 0.25) (layer "F.Cu") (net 6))
 (segment (start 143.129 84.582) (end 144.018 85.471) (width 0.25) (layer "F.Cu") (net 6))
 (segment (start 144.018 85.471) (end 144.653 85.471) (width 0.25) (layer "F.Cu") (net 6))
 (segment (start 147.066 87.376) (end 147.066 93.98) (width 0.25) (layer "F.Cu") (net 6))
 (segment (start 149.98 95.243) (end 149.98 96.774) (width 0.25) (layer "F.Cu") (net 6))
 (segment (start 147.193 94.107) (end 148.844 94.107) (width 0.25) (layer "F.Cu") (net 6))
 (segment (start 124.714 79.756) (end 129.794 79.756) (width 0.25) (layer "F.Cu") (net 7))
 (segment (start 123.952 81.804) (end 123.952 80.518) (width 0.25) (layer "F.Cu") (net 7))
 (segment (start 129.794 79.756) (end 130.556 80.518) (width 0.25) (layer "F.Cu") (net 7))
 (segment (start 131.172 86.214) (end 134.998 86.214) (width 0.25) (layer "F.Cu") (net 7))
 (segment (start 130.556 80.518) (end 130.556 85.598) (width 0.25) (layer "F.Cu") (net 7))
 (segment (start 130.556 85.598) (end 131.172 86.214) (width 0.25) (layer "F.Cu") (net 7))
 (segment (start 123.952 80.518) (end 124.714 79.756) (width 0.25) (layer "F.Cu") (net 7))
 (segment (start 144.272 78.74) (end 147.066 81.534) (width 0.5) (layer "F.Cu") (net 1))
 (segment (start 124.206 78.74) (end 144.272 78.74) (width 0.5) (layer "F.Cu") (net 1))
 (segment (start 124.2695 89.4715) (end 124.206 89.408) (width 0.5) (layer "F.Cu") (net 1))
 (segment (start 124.206 89.408) (end 124.206 85.217) (width 0.5) (layer "F.Cu") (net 1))
 (segment (start 122.428 83.82) (end 122.428 80.518) (width 0.5) (layer "F.Cu") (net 1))
 (segment (start 122.3905 83.8575) (end 122.428 83.82) (width 0.5) (layer "F.Cu") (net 1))
 (segment (start 122.428 80.518) (end 124.206 78.74) (width 0.5) (layer "F.Cu") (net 1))
 (segment (start 121.285 85.217) (end 120.904 84.836) (width 0.5) (layer "F.Cu") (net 1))
 (segment (start 124.206 85.217) (end 121.285 85.217) (width 0.5) (layer "F.Cu") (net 1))
 (segment (start 120.904 84.836) (end 120.904 83.8575) (width 0.5) (layer "F.Cu") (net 1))
 (segment (start 147.066 81.534) (end 149.98 81.534) (width 0.5) (layer "F.Cu") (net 1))
 (segment (start 125.857 89.4715) (end 124.2695 89.4715) (width 0.5) (layer "F.Cu") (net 1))
 (segment (start 120.904 83.8575) (end 122.3905 83.8575) (width 0.5) (layer "F.Cu") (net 1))
 (segment (start 115.8025 87.884) (end 115.8025 85.598) (width 0.5) (layer "F.Cu") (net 3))
 (segment (start 113.284 84.836) (end 107.188 84.836) (width 0.5) (layer "F.Cu") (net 3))
 (segment (start 114.046 85.598) (end 113.284 84.836) (width 0.5) (layer "F.Cu") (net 3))
 (segment (start 107.188 84.836) (end 106.426 85.598) (width 0.5) (layer "F.Cu") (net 3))
 (segment (start 106.426 85.598) (end 106.426 87.604) (width 0.5) (layer "F.Cu") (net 3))
 (segment (start 115.8025 85.598) (end 114.046 85.598) (width 0.5) (layer "F.Cu") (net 3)))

